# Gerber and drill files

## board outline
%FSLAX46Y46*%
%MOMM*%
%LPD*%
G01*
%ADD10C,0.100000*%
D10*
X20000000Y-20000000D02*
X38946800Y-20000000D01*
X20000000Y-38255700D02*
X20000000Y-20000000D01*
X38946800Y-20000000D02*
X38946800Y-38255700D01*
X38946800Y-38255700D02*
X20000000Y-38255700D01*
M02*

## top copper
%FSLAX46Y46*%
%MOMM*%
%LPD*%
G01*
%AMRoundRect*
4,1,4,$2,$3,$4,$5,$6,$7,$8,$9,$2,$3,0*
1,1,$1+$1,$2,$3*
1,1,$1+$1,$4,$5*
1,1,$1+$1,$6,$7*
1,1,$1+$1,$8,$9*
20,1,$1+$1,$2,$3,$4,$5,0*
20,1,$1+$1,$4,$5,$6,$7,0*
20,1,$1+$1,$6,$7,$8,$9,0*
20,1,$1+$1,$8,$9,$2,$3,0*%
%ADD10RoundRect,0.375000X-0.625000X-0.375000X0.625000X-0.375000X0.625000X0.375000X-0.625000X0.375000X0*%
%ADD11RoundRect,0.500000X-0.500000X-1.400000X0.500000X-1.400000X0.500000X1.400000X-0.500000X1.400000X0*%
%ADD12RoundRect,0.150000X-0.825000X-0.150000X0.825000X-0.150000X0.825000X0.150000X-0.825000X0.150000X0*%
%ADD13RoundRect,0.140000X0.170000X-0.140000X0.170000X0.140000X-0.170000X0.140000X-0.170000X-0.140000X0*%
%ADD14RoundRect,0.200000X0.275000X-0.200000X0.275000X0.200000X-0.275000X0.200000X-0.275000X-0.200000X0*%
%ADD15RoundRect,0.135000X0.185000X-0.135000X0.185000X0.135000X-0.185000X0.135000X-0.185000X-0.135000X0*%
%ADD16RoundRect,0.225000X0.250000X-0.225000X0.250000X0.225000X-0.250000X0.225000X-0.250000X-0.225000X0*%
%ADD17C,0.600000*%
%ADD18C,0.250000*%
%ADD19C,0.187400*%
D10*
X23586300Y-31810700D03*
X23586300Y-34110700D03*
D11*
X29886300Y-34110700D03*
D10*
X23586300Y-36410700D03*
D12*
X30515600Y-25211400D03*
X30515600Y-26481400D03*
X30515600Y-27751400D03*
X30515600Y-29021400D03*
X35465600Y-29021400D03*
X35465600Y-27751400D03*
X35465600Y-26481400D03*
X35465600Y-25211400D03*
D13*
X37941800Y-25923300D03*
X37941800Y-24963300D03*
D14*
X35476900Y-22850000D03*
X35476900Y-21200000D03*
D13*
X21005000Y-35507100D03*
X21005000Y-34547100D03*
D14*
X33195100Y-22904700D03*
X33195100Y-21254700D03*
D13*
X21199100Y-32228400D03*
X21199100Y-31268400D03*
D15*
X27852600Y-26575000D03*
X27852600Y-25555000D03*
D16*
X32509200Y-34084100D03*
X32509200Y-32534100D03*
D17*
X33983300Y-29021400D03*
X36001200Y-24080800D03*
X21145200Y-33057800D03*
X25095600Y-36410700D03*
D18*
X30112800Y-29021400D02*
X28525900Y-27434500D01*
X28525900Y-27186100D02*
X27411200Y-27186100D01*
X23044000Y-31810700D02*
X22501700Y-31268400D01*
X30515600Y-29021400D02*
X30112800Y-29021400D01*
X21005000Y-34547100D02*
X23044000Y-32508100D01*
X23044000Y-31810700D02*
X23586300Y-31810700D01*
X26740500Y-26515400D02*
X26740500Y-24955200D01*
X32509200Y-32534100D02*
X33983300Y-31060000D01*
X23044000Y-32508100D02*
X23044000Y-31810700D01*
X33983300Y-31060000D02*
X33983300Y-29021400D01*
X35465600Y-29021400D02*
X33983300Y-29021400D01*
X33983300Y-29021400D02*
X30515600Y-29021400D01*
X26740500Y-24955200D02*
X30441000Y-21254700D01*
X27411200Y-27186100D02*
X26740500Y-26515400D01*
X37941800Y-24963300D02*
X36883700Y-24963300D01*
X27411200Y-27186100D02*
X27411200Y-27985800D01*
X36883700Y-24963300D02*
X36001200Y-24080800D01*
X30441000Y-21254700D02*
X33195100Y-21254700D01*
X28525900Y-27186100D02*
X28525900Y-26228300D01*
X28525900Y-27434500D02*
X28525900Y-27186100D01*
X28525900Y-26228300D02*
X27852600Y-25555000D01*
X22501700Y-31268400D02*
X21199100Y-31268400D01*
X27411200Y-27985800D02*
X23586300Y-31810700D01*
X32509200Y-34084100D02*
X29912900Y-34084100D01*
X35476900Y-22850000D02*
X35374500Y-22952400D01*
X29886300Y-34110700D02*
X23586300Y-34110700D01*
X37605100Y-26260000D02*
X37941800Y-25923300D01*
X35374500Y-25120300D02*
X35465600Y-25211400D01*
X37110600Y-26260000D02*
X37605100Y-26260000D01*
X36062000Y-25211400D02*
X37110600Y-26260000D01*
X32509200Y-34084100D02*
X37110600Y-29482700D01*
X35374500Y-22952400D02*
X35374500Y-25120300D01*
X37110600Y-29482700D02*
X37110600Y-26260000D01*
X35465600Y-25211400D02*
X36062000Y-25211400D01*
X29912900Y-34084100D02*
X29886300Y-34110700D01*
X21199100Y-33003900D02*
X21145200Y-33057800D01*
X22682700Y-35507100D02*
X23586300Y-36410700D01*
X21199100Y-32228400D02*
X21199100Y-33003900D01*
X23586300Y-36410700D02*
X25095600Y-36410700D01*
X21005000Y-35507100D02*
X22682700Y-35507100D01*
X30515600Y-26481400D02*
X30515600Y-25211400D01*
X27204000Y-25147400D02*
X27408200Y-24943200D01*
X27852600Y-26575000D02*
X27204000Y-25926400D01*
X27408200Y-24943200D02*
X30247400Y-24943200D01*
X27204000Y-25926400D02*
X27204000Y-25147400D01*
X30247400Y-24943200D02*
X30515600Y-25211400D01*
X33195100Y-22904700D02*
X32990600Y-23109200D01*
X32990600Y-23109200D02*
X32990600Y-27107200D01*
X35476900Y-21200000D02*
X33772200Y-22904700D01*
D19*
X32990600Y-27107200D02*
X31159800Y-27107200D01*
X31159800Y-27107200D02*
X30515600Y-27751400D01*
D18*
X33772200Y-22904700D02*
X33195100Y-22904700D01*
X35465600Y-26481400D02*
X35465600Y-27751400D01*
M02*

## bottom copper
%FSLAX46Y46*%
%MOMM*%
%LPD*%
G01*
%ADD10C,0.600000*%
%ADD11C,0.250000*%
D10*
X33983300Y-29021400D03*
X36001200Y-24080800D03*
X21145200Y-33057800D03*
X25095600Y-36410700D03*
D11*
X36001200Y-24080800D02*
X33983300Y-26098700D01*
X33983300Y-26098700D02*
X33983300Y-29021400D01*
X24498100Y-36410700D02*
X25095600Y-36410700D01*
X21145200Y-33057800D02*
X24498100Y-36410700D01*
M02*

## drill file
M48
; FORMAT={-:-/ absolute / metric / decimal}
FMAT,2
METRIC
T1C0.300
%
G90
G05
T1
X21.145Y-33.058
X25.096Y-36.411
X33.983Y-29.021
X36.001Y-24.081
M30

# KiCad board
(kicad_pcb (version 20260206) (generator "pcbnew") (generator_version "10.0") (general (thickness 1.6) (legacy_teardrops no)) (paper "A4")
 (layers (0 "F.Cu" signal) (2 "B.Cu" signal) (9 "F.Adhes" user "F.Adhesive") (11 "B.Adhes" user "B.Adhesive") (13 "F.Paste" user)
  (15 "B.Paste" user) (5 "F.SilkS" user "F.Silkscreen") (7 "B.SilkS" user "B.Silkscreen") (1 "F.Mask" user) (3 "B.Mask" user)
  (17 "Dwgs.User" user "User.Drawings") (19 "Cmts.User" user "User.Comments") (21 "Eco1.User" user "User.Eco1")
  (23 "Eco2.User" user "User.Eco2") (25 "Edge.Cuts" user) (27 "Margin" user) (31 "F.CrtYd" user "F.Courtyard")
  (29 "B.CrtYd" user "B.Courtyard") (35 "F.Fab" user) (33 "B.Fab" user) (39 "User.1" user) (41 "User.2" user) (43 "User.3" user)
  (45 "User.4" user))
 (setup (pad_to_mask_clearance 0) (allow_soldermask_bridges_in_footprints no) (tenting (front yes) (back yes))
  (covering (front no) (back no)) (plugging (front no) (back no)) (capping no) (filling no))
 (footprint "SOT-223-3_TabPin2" (layer "F.Cu") (at 26.7363 34.1107)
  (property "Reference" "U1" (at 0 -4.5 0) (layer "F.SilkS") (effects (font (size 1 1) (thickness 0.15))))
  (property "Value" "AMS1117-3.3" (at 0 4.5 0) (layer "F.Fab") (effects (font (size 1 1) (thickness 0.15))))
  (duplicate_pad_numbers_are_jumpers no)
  (pad "1" smd roundrect (at -3.15 -2.3) (size 2 1.5) (layers "F.Cu" "F.Mask" "F.Paste") (roundrect_rratio 0.25) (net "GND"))
  (pad "2" smd roundrect (at -3.15 0) (size 2 1.5) (layers "F.Cu" "F.Mask" "F.Paste") (roundrect_rratio 0.25) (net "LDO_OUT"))
  (pad "2" smd roundrect (at 3.15 0) (size 2 3.8) (layers "F.Cu" "F.Mask" "F.Paste") (roundrect_rratio 0.25) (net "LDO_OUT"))
  (pad "3" smd roundrect (at -3.15 2.3) (size 2 1.5) (layers "F.Cu" "F.Mask" "F.Paste") (roundrect_rratio 0.25) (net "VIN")))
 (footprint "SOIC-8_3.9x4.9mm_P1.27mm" (layer "F.Cu") (at 32.9906 27.1164)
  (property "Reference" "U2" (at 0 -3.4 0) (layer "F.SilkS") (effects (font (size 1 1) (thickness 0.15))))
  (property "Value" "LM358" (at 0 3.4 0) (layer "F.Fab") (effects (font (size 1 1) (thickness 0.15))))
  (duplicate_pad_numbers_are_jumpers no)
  (pad "1" smd roundrect (at -2.475 -1.905) (size 1.95 0.6) (layers "F.Cu" "F.Mask" "F.Paste") (roundrect_rratio 0.25) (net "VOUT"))
  (pad "2" smd roundrect (at -2.475 -0.635) (size 1.95 0.6) (layers "F.Cu" "F.Mask" "F.Paste") (roundrect_rratio 0.25) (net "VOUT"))
  (pad "3" smd roundrect (at -2.475 0.635) (size 1.95 0.6) (layers "F.Cu" "F.Mask" "F.Paste") (roundrect_rratio 0.25) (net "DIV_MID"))
  (pad "4" smd roundrect (at -2.475 1.905) (size 1.95 0.6) (layers "F.Cu" "F.Mask" "F.Paste") (roundrect_rratio 0.25) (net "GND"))
  (pad "5" smd roundrect (at 2.475 1.905) (size 1.95 0.6) (layers "F.Cu" "F.Mask" "F.Paste") (roundrect_rratio 0.25) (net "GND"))
  (pad "6" smd roundrect (at 2.475 0.635) (size 1.95 0.6) (layers "F.Cu" "F.Mask" "F.Paste") (roundrect_rratio 0.25) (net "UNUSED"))
  (pad "7" smd roundrect (at 2.475 -0.635) (size 1.95 0.6) (layers "F.Cu" "F.Mask" "F.Paste") (roundrect_rratio 0.25) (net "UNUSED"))
  (pad "8" smd roundrect (at 2.475 -1.905) (size 1.95 0.6) (layers "F.Cu" "F.Mask" "F.Paste") (roundrect_rratio 0.25) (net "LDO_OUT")))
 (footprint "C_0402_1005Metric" (layer "F.Cu") (at 37.9418 25.4433 90)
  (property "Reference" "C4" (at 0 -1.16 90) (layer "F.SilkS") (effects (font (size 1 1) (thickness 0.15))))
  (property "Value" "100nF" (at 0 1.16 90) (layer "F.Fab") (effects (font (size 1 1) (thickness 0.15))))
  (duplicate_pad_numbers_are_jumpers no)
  (pad "1" smd roundrect (at -0.48 0 90) (size 0.56 0.62) (layers "F.Cu" "F.Mask" "F.Paste") (roundrect_rratio 0.25) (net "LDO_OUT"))
  (pad "2" smd roundrect (at 0.48 0 90) (size 0.56 0.62) (layers "F.Cu" "F.Mask" "F.Paste") (roundrect_rratio 0.25) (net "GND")))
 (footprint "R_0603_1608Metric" (layer "F.Cu") (at 35.4769 22.025 90)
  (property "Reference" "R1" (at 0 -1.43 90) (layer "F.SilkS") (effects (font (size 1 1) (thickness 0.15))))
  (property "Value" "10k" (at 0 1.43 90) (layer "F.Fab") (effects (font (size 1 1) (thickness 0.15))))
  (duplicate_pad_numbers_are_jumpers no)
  (pad "1" smd roundrect (at -0.825 0 90) (size 0.8 0.95) (layers "F.Cu" "F.Mask" "F.Paste") (roundrect_rratio 0.25) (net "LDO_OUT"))
  (pad "2" smd roundrect (at 0.825 0 90) (size 0.8 0.95) (layers "F.Cu" "F.Mask" "F.Paste") (roundrect_rratio 0.25) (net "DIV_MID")))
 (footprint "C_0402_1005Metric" (layer "F.Cu") (at 21.005 35.0271 90)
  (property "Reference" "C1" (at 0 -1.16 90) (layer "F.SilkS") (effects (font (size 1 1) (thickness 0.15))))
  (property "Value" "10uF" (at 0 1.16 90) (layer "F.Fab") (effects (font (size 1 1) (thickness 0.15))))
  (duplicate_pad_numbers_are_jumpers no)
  (pad "1" smd roundrect (at -0.48 0 90) (size 0.56 0.62) (layers "F.Cu" "F.Mask" "F.Paste") (roundrect_rratio 0.25) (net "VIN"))
  (pad "2" smd roundrect (at 0.48 0 90) (size 0.56 0.62) (layers "F.Cu" "F.Mask" "F.Paste") (roundrect_rratio 0.25) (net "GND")))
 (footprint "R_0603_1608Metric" (layer "F.Cu") (at 33.1951 22.0797 90)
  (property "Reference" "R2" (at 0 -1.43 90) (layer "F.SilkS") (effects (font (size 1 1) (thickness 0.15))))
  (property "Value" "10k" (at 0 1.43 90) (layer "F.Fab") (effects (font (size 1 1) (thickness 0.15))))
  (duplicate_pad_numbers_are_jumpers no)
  (pad "1" smd roundrect (at -0.825 0 90) (size 0.8 0.95) (layers "F.Cu" "F.Mask" "F.Paste") (roundrect_rratio 0.25) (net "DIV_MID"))
  (pad "2" smd roundrect (at 0.825 0 90) (size 0.8 0.95) (layers "F.Cu" "F.Mask" "F.Paste") (roundrect_rratio 0.25) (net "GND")))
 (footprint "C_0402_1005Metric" (layer "F.Cu") (at 21.1991 31.7484 90)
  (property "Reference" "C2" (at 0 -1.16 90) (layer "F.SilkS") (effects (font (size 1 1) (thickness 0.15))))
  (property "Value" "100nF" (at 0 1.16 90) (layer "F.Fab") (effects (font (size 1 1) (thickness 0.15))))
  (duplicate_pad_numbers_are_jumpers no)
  (pad "1" smd roundrect (at -0.48 0 90) (size 0.56 0.62) (layers "F.Cu" "F.Mask" "F.Paste") (roundrect_rratio 0.25) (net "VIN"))
  (pad "2" smd roundrect (at 0.48 0 90) (size 0.56 0.62) (layers "F.Cu" "F.Mask" "F.Paste") (roundrect_rratio 0.25) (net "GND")))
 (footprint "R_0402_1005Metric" (layer "F.Cu") (at 27.8526 26.065 90)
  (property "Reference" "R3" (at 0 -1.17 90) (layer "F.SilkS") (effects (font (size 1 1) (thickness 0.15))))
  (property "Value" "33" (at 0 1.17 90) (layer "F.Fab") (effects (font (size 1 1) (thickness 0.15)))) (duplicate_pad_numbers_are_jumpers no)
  (pad "1" smd roundrect (at -0.51 0 90) (size 0.54 0.64) (layers "F.Cu" "F.Mask" "F.Paste") (roundrect_rratio 0.25) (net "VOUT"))
  (pad "2" smd roundrect (at 0.51 0 90) (size 0.54 0.64) (layers "F.Cu" "F.Mask" "F.Paste") (roundrect_rratio 0.25) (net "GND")))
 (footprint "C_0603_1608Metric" (layer "F.Cu") (at 32.5092 33.3091 90)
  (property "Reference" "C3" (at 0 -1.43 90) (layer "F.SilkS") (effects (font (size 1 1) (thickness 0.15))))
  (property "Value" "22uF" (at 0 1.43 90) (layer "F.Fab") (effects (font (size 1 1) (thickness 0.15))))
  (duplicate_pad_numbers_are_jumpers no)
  (pad "1" smd roundrect (at -0.775 0 90) (size 0.9 0.95) (layers "F.Cu" "F.Mask" "F.Paste") (roundrect_rratio 0.25) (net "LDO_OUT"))
  (pad "2" smd roundrect (at 0.775 0 90) (size 0.9 0.95) (layers "F.Cu" "F.Mask" "F.Paste") (roundrect_rratio 0.25) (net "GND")))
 (gr_line (start 20 20) (end 38.9468 20) (stroke (width 0.1) (type default)) (layer "Edge.Cuts"))
 (gr_line (start 20 38.2557) (end 20 20) (stroke (width 0.1) (type default)) (layer "Edge.Cuts"))
 (gr_line (start 38.9468 20) (end 38.9468 38.2557) (stroke (width 0.1) (type default)) (layer "Edge.Cuts"))
 (gr_line (start 38.9468 38.2557) (end 20 38.2557) (stroke (width 0.1) (type default)) (layer "Edge.Cuts"))
 (segment (start 30.1128 29.0214) (end 28.5259 27.4345) (width 0.25) (layer "F.Cu") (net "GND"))
 (segment (start 28.5259 27.1861) (end 27.4112 27.1861) (width 0.25) (layer "F.Cu") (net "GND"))
 (segment (start 23.044 31.8107) (end 22.5017 31.2684) (width 0.25) (layer "F.Cu") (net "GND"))
 (segment (start 30.5156 29.0214) (end 30.1128 29.0214) (width 0.25) (layer "F.Cu") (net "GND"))
 (segment (start 21.005 34.5471) (end 23.044 32.5081) (width 0.25) (layer "F.Cu") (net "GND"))
 (segment (start 23.044 31.8107) (end 23.5863 31.8107) (width 0.25) (layer "F.Cu") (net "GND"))
 (segment (start 26.7405 26.5154) (end 26.7405 24.9552) (width 0.25) (layer "F.Cu") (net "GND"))
 (segment (start 32.5092 32.5341) (end 33.9833 31.06) (width 0.25) (layer "F.Cu") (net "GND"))
 (segment (start 23.044 32.5081) (end 23.044 31.8107) (width 0.25) (layer "F.Cu") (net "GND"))
 (segment (start 33.9833 31.06) (end 33.9833 29.0214) (width 0.25) (layer "F.Cu") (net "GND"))
 (segment (start 35.4656 29.0214) (end 33.9833 29.0214) (width 0.25) (layer "F.Cu") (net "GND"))
 (segment (start 33.9833 29.0214) (end 30.5156 29.0214) (width 0.25) (layer "F.Cu") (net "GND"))
 (segment (start 26.7405 24.9552) (end 30.441 21.2547) (width 0.25) (layer "F.Cu") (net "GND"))
 (segment (start 27.4112 27.1861) (end 26.7405 26.5154) (width 0.25) (layer "F.Cu") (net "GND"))
 (segment (start 37.9418 24.9633) (end 36.8837 24.9633) (width 0.25) (layer "F.Cu") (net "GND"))
 (segment (start 27.4112 27.1861) (end 27.4112 27.9858) (width 0.25) (layer "F.Cu") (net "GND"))
 (segment (start 36.8837 24.9633) (end 36.0012 24.0808) (width 0.25) (layer "F.Cu") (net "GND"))
 (segment (start 30.441 21.2547) (end 33.1951 21.2547) (width 0.25) (layer "F.Cu") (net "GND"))
 (segment (start 28.5259 27.1861) (end 28.5259 26.2283) (width 0.25) (layer "F.Cu") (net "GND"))
 (segment (start 28.5259 27.4345) (end 28.5259 27.1861) (width 0.25) (layer "F.Cu") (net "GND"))
 (segment (start 28.5259 26.2283) (end 27.8526 25.555) (width 0.25) (layer "F.Cu") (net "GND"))
 (segment (start 22.5017 31.2684) (end 21.1991 31.2684) (width 0.25) (layer "F.Cu") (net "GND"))
 (segment (start 27.4112 27.9858) (end 23.5863 31.8107) (width 0.25) (layer "F.Cu") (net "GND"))
 (via (at 33.9833 29.0214) (size 0.6) (drill 0.3) (layers "F.Cu" "B.Cu") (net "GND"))
 (via (at 36.0012 24.0808) (size 0.6) (drill 0.3) (layers "F.Cu" "B.Cu") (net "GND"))
 (segment (start 36.0012 24.0808) (end 33.9833 26.0987) (width 0.25) (layer "B.Cu") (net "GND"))
 (segment (start 33.9833 26.0987) (end 33.9833 29.0214) (width 0.25) (layer "B.Cu") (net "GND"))
 (segment (start 32.5092 34.0841) (end 29.9129 34.0841) (width 0.25) (layer "F.Cu") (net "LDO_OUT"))
 (segment (start 35.4769 22.85) (end 35.3745 22.9524) (width 0.25) (layer "F.Cu") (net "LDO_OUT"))
 (segment (start 29.8863 34.1107) (end 23.5863 34.1107) (width 0.25) (layer "F.Cu") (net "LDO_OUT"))
 (segment (start 37.6051 26.26) (end 37.9418 25.9233) (width 0.25) (layer "F.Cu") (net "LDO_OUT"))
 (segment (start 35.3745 25.1203) (end 35.4656 25.2114) (width 0.25) (layer "F.Cu") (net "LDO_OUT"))
 (segment (start 37.1106 26.26) (end 37.6051 26.26) (width 0.25) (layer "F.Cu") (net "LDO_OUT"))
 (segment (start 36.062 25.2114) (end 37.1106 26.26) (width 0.25) (layer "F.Cu") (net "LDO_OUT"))
 (segment (start 32.5092 34.0841) (end 37.1106 29.4827) (width 0.25) (layer "F.Cu") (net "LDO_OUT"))
 (segment (start 35.3745 22.9524) (end 35.3745 25.1203) (width 0.25) (layer "F.Cu") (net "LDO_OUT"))
 (segment (start 37.1106 29.4827) (end 37.1106 26.26) (width 0.25) (layer "F.Cu") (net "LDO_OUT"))
 (segment (start 35.4656 25.2114) (end 36.062 25.2114) (width 0.25) (layer "F.Cu") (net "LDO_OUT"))
 (segment (start 29.9129 34.0841) (end 29.8863 34.1107) (width 0.25) (layer "F.Cu") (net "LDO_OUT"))
 (segment (start 21.1991 33.0039) (end 21.1452 33.0578) (width 0.25) (layer "F.Cu") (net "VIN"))
 (segment (start 22.6827 35.5071) (end 23.5863 36.4107) (width 0.25) (layer "F.Cu") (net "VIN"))
 (segment (start 21.1991 32.2284) (end 21.1991 33.0039) (width 0.25) (layer "F.Cu") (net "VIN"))
 (segment (start 23.5863 36.4107) (end 25.0956 36.4107) (width 0.25) (layer "F.Cu") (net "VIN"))
 (segment (start 21.005 35.5071) (end 22.6827 35.5071) (width 0.25) (layer "F.Cu") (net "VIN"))
 (via (at 21.1452 33.0578) (size 0.6) (drill 0.3) (layers "F.Cu" "B.Cu") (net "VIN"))
 (via (at 25.0956 36.4107) (size 0.6) (drill 0.3) (layers "F.Cu" "B.Cu") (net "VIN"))
 (segment (start 24.4981 36.4107) (end 25.0956 36.4107) (width 0.25) (layer "B.Cu") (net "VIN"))
 (segment (start 21.1452 33.0578) (end 24.4981 36.4107) (width 0.25) (layer "B.Cu") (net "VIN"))
 (segment (start 30.5156 26.4814) (end 30.5156 25.2114) (width 0.25) (layer "F.Cu") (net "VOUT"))
 (segment (start 27.204 25.1474) (end 27.4082 24.9432) (width 0.25) (layer "F.Cu") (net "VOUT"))
 (segment (start 27.8526 26.575) (end 27.204 25.9264) (width 0.25) (layer "F.Cu") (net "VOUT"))
 (segment (start 27.4082 24.9432) (end 30.2474 24.9432) (width 0.25) (layer "F.Cu") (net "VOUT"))
 (segment (start 27.204 25.9264) (end 27.204 25.1474) (width 0.25) (layer "F.Cu") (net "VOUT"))
 (segment (start 30.2474 24.9432) (end 30.5156 25.2114) (width 0.25) (layer "F.Cu") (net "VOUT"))
 (segment (start 33.1951 22.9047) (end 32.9906 23.1092) (width 0.25) (layer "F.Cu") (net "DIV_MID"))
 (segment (start 32.9906 23.1092) (end 32.9906 27.1072) (width 0.25) (layer "F.Cu") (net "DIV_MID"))
 (segment (start 35.4769 21.2) (end 33.7722 22.9047) (width 0.25) (layer "F.Cu") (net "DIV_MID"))
 (segment (start 32.9906 27.1072) (end 31.1598 27.1072) (width 0.1874) (layer "F.Cu") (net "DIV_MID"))
 (segment (start 31.1598 27.1072) (end 30.5156 27.7514) (width 0.1874) (layer "F.Cu") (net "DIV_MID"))
 (segment (start 33.7722 22.9047) (end 33.1951 22.9047) (width 0.25) (layer "F.Cu") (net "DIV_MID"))
 (segment (start 35.4656 26.4814) (end 35.4656 27.7514) (width 0.25) (layer "F.Cu") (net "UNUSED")))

